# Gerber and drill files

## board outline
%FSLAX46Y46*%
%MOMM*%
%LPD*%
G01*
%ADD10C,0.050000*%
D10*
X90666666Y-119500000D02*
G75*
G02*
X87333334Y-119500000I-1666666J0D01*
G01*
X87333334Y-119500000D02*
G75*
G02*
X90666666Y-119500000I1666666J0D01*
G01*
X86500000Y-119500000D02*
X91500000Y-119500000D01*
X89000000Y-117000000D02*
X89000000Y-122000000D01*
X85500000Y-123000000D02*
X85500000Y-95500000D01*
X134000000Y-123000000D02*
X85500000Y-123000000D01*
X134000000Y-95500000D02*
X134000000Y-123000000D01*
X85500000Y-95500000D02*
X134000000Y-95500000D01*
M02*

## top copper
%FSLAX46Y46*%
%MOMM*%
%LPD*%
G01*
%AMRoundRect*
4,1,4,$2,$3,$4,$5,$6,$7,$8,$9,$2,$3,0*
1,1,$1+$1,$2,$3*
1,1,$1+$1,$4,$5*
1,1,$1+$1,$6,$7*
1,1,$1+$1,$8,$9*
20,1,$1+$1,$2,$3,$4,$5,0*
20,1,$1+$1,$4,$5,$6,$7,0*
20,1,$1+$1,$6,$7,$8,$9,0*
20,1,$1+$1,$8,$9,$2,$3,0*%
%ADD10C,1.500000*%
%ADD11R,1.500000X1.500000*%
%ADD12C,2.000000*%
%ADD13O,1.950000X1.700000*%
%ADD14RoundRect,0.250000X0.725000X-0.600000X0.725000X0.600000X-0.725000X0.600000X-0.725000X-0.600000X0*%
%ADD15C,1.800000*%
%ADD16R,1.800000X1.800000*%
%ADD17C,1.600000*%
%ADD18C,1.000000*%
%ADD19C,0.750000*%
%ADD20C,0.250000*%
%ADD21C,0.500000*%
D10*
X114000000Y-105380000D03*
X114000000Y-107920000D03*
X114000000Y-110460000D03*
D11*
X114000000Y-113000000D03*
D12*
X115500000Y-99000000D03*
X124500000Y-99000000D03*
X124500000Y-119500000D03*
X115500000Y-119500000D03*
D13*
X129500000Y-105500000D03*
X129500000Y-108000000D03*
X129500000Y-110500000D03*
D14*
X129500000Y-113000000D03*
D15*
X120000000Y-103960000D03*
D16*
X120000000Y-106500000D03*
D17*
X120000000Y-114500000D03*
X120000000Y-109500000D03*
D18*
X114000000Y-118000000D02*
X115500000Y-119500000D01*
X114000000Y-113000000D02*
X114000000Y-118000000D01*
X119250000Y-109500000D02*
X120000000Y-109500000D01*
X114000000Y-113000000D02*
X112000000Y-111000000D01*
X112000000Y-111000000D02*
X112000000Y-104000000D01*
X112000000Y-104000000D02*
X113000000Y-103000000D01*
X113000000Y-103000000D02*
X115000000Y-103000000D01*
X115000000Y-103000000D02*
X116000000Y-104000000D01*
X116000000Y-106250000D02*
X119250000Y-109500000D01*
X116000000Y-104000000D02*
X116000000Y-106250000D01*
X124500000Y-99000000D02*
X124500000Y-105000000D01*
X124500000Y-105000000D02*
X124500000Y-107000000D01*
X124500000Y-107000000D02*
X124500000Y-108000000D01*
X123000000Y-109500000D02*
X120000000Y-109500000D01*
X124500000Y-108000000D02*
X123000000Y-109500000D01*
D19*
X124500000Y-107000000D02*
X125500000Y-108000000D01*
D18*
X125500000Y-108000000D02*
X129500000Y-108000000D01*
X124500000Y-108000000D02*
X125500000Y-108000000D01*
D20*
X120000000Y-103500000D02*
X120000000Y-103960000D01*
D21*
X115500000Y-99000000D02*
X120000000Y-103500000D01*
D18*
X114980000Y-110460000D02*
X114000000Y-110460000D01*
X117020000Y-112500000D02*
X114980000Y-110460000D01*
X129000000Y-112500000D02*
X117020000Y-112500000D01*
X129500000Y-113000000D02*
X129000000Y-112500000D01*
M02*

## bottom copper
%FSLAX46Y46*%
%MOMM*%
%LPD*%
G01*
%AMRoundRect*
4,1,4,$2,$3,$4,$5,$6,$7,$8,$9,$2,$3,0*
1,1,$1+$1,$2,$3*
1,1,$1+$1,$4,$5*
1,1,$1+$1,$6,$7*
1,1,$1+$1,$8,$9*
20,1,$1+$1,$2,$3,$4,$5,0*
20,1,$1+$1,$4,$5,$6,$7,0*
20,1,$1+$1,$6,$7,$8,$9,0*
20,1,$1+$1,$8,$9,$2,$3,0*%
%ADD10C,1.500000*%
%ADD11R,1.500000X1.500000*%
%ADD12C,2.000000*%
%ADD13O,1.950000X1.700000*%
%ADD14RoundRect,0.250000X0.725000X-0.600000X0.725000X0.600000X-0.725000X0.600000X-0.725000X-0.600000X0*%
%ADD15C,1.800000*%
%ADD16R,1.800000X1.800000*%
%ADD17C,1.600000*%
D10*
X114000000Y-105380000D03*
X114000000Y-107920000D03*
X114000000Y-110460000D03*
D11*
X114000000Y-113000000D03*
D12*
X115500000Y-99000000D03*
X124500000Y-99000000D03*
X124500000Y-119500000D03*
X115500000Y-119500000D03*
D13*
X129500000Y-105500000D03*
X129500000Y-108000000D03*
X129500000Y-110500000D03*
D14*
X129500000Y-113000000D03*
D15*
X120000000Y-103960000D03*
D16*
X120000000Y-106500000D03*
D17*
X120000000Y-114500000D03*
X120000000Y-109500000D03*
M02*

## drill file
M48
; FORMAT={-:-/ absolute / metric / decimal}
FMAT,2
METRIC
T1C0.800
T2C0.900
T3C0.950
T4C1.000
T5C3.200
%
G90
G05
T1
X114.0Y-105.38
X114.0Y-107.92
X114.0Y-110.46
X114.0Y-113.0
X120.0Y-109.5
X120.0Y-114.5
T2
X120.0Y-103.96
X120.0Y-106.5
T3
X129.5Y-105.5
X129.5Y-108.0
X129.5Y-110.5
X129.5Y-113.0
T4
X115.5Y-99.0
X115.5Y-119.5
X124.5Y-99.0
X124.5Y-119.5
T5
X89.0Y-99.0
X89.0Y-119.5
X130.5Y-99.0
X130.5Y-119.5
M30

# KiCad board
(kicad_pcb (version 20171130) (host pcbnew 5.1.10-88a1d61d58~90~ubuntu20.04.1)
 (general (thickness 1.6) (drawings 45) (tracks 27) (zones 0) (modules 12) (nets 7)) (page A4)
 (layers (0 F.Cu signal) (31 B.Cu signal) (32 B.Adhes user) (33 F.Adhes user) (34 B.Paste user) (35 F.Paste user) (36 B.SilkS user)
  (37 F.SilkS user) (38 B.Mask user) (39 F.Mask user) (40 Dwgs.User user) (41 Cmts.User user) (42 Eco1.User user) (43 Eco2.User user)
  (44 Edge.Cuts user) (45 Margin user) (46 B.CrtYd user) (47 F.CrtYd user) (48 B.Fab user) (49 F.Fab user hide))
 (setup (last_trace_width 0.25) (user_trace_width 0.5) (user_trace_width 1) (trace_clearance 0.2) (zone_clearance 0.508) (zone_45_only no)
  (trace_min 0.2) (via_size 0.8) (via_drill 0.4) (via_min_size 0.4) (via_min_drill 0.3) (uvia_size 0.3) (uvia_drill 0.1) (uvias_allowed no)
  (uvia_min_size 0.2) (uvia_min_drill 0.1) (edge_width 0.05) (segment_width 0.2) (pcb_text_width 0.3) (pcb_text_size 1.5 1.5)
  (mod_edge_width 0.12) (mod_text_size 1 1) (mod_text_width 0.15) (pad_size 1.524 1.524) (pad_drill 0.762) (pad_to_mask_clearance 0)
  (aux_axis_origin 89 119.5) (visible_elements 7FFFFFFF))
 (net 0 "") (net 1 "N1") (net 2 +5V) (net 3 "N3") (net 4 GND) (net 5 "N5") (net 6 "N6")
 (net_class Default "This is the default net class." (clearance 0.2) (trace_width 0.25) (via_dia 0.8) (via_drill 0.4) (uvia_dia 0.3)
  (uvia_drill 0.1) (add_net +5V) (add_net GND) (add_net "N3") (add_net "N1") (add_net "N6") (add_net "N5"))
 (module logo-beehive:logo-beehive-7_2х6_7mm (layer F.Cu) (at 98 119)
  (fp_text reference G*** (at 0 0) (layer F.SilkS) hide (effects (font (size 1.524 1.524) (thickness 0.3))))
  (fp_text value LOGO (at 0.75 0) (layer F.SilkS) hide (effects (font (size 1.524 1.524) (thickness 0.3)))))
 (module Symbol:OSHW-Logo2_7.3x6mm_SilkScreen (layer F.Cu) (at 106.5 119.5)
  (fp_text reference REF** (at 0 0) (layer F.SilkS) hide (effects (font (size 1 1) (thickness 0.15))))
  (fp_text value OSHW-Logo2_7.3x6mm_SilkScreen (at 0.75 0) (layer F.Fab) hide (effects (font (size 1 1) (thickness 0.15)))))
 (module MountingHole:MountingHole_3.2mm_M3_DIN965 (layer F.Cu) (at 89 119.5 180)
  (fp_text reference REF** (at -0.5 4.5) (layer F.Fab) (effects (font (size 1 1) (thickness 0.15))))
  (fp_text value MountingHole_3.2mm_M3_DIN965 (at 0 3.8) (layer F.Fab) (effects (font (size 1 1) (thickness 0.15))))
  (pad 1 np_thru_hole circle (at 0 0 180) (size 3.2 3.2) (drill 3.2) (layers *.Cu *.Mask)))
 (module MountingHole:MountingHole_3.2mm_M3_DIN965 (layer F.Cu) (at 89 99 90)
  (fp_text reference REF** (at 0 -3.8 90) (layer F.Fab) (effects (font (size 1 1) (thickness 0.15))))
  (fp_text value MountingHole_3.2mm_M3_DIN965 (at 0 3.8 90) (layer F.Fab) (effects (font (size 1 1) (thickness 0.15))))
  (pad 1 np_thru_hole circle (at 0 0 90) (size 3.2 3.2) (drill 3.2) (layers *.Cu *.Mask)))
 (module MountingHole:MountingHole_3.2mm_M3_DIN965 (layer F.Cu) (at 130.5 119.5)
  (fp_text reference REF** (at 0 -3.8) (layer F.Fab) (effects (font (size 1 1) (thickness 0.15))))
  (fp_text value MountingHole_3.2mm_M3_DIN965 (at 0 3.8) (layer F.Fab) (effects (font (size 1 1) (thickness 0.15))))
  (pad 1 np_thru_hole circle (at 0 0) (size 3.2 3.2) (drill 3.2) (layers *.Cu *.Mask)))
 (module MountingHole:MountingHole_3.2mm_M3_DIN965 (layer F.Cu) (at 130.5 99)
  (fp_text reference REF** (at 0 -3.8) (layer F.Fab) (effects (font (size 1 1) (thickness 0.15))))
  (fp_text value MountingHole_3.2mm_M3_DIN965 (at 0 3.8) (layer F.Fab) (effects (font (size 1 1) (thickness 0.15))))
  (pad 1 np_thru_hole circle (at 0 0) (size 3.2 3.2) (drill 3.2) (layers *.Cu *.Mask)))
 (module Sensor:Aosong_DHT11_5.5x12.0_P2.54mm (layer F.Cu) (at 114 113 180)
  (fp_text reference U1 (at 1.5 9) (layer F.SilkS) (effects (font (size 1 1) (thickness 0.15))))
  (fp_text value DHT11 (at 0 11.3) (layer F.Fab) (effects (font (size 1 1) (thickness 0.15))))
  (pad 4 thru_hole circle (at 0 7.62 180) (size 1.5 1.5) (drill 0.8) (layers *.Cu *.Mask))
  (pad 3 thru_hole circle (at 0 5.08 180) (size 1.5 1.5) (drill 0.8) (layers *.Cu *.Mask))
  (pad 2 thru_hole circle (at 0 2.54 180) (size 1.5 1.5) (drill 0.8) (layers *.Cu *.Mask) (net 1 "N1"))
  (pad 1 thru_hole rect (at 0 0 180) (size 1.5 1.5) (drill 0.8) (layers *.Cu *.Mask) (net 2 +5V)))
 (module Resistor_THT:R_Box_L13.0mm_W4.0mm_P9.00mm (layer F.Cu) (at 124.5 99 180)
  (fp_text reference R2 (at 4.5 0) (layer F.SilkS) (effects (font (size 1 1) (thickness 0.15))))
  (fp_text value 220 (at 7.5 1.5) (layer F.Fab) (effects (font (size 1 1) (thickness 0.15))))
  (pad 2 thru_hole circle (at 9 0 180) (size 2 2) (drill 1) (layers *.Cu *.Mask) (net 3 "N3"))
  (pad 1 thru_hole circle (at 0 0 180) (size 2 2) (drill 1) (layers *.Cu *.Mask) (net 2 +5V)))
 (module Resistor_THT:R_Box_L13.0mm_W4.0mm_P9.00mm (layer F.Cu) (at 115.5 119.5)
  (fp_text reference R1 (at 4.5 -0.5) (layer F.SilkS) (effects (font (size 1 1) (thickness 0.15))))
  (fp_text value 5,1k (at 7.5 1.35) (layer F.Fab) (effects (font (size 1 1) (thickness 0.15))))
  (pad 2 thru_hole circle (at 9 0) (size 2 2) (drill 1) (layers *.Cu *.Mask))
  (pad 1 thru_hole circle (at 0 0) (size 2 2) (drill 1) (layers *.Cu *.Mask) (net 2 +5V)))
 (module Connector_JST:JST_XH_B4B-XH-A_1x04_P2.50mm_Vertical (layer F.Cu) (at 129.5 113 90)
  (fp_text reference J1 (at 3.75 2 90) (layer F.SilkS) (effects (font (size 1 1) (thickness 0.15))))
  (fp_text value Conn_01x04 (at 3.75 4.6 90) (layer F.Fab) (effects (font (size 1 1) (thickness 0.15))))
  (pad 4 thru_hole oval (at 7.5 0 90) (size 1.7 1.95) (drill 0.95) (layers *.Cu *.Mask))
  (pad 3 thru_hole oval (at 5 0 90) (size 1.7 1.95) (drill 0.95) (layers *.Cu *.Mask) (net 2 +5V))
  (pad 2 thru_hole oval (at 2.5 0 90) (size 1.7 1.95) (drill 0.95) (layers *.Cu *.Mask))
  (pad 1 thru_hole roundrect (at 0 0 90) (size 1.7 1.95) (drill 0.95) (layers *.Cu *.Mask) (roundrect_rratio 0.1470588235294118)
   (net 1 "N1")))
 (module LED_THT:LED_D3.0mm (layer F.Cu) (at 120 106.5 90)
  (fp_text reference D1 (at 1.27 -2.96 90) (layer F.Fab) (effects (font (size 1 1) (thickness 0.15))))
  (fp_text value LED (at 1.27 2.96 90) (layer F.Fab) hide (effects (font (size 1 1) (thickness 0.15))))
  (pad 2 thru_hole circle (at 2.54 0 90) (size 1.8 1.8) (drill 0.9) (layers *.Cu *.Mask) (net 3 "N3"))
  (pad 1 thru_hole rect (at 0 0 90) (size 1.8 1.8) (drill 0.9) (layers *.Cu *.Mask)))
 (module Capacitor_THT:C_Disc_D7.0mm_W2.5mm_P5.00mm (layer F.Cu) (at 120 109.5 270)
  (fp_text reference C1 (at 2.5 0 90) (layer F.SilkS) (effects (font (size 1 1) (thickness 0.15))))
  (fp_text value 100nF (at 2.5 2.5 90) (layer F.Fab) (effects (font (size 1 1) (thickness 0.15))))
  (pad 2 thru_hole circle (at 5 0 270) (size 1.6 1.6) (drill 0.8) (layers *.Cu *.Mask))
  (pad 1 thru_hole circle (at 0 0 270) (size 1.6 1.6) (drill 0.8) (layers *.Cu *.Mask) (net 2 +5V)))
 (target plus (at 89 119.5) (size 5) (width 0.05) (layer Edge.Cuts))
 (gr_line (start 85.5 123) (end 85.5 95.5) (layer Edge.Cuts) (width 0.05))
 (gr_line (start 134 123) (end 85.5 123) (layer Edge.Cuts) (width 0.05))
 (gr_line (start 134 95.5) (end 134 123) (layer Edge.Cuts) (width 0.05))
 (gr_line (start 85.5 95.5) (end 134 95.5) (layer Edge.Cuts) (width 0.05))
 (segment (start 114 118) (end 115.5 119.5) (width 1) (layer F.Cu) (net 2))
 (segment (start 114 113) (end 114 118) (width 1) (layer F.Cu) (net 2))
 (segment (start 119.25 109.5) (end 120 109.5) (width 1) (layer F.Cu) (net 2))
 (segment (start 114 113) (end 112 111) (width 1) (layer F.Cu) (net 2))
 (segment (start 112 111) (end 112 104) (width 1) (layer F.Cu) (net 2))
 (segment (start 112 104) (end 113 103) (width 1) (layer F.Cu) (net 2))
 (segment (start 113 103) (end 115 103) (width 1) (layer F.Cu) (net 2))
 (segment (start 115 103) (end 116 104) (width 1) (layer F.Cu) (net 2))
 (segment (start 116 106.25) (end 119.25 109.5) (width 1) (layer F.Cu) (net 2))
 (segment (start 116 104) (end 116 106.25) (width 1) (layer F.Cu) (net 2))
 (segment (start 124.5 99) (end 124.5 105) (width 1) (layer F.Cu) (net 2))
 (segment (start 124.5 105) (end 124.5 107) (width 1) (layer F.Cu) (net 2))
 (segment (start 124.5 107) (end 124.5 108) (width 1) (layer F.Cu) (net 2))
 (segment (start 123 109.5) (end 120 109.5) (width 1) (layer F.Cu) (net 2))
 (segment (start 124.5 108) (end 123 109.5) (width 1) (layer F.Cu) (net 2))
 (segment (start 124.5 107) (end 125.5 108) (width 0.75) (layer F.Cu) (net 2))
 (segment (start 125.5 108) (end 129.5 108) (width 1) (layer F.Cu) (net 2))
 (segment (start 124.5 108) (end 125.5 108) (width 1) (layer F.Cu) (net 2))
 (segment (start 120 103.5) (end 120 103.96) (width 0.25) (layer F.Cu) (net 3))
 (segment (start 115.5 99) (end 120 103.5) (width 0.5) (layer F.Cu) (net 3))
 (segment (start 114.98 110.46) (end 114 110.46) (width 1) (layer F.Cu) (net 1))
 (segment (start 117.02 112.5) (end 114.98 110.46) (width 1) (layer F.Cu) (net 1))
 (segment (start 129 112.5) (end 117.02 112.5) (width 1) (layer F.Cu) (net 1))
 (segment (start 129.5 113) (end 129 112.5) (width 1) (layer F.Cu) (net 1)))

